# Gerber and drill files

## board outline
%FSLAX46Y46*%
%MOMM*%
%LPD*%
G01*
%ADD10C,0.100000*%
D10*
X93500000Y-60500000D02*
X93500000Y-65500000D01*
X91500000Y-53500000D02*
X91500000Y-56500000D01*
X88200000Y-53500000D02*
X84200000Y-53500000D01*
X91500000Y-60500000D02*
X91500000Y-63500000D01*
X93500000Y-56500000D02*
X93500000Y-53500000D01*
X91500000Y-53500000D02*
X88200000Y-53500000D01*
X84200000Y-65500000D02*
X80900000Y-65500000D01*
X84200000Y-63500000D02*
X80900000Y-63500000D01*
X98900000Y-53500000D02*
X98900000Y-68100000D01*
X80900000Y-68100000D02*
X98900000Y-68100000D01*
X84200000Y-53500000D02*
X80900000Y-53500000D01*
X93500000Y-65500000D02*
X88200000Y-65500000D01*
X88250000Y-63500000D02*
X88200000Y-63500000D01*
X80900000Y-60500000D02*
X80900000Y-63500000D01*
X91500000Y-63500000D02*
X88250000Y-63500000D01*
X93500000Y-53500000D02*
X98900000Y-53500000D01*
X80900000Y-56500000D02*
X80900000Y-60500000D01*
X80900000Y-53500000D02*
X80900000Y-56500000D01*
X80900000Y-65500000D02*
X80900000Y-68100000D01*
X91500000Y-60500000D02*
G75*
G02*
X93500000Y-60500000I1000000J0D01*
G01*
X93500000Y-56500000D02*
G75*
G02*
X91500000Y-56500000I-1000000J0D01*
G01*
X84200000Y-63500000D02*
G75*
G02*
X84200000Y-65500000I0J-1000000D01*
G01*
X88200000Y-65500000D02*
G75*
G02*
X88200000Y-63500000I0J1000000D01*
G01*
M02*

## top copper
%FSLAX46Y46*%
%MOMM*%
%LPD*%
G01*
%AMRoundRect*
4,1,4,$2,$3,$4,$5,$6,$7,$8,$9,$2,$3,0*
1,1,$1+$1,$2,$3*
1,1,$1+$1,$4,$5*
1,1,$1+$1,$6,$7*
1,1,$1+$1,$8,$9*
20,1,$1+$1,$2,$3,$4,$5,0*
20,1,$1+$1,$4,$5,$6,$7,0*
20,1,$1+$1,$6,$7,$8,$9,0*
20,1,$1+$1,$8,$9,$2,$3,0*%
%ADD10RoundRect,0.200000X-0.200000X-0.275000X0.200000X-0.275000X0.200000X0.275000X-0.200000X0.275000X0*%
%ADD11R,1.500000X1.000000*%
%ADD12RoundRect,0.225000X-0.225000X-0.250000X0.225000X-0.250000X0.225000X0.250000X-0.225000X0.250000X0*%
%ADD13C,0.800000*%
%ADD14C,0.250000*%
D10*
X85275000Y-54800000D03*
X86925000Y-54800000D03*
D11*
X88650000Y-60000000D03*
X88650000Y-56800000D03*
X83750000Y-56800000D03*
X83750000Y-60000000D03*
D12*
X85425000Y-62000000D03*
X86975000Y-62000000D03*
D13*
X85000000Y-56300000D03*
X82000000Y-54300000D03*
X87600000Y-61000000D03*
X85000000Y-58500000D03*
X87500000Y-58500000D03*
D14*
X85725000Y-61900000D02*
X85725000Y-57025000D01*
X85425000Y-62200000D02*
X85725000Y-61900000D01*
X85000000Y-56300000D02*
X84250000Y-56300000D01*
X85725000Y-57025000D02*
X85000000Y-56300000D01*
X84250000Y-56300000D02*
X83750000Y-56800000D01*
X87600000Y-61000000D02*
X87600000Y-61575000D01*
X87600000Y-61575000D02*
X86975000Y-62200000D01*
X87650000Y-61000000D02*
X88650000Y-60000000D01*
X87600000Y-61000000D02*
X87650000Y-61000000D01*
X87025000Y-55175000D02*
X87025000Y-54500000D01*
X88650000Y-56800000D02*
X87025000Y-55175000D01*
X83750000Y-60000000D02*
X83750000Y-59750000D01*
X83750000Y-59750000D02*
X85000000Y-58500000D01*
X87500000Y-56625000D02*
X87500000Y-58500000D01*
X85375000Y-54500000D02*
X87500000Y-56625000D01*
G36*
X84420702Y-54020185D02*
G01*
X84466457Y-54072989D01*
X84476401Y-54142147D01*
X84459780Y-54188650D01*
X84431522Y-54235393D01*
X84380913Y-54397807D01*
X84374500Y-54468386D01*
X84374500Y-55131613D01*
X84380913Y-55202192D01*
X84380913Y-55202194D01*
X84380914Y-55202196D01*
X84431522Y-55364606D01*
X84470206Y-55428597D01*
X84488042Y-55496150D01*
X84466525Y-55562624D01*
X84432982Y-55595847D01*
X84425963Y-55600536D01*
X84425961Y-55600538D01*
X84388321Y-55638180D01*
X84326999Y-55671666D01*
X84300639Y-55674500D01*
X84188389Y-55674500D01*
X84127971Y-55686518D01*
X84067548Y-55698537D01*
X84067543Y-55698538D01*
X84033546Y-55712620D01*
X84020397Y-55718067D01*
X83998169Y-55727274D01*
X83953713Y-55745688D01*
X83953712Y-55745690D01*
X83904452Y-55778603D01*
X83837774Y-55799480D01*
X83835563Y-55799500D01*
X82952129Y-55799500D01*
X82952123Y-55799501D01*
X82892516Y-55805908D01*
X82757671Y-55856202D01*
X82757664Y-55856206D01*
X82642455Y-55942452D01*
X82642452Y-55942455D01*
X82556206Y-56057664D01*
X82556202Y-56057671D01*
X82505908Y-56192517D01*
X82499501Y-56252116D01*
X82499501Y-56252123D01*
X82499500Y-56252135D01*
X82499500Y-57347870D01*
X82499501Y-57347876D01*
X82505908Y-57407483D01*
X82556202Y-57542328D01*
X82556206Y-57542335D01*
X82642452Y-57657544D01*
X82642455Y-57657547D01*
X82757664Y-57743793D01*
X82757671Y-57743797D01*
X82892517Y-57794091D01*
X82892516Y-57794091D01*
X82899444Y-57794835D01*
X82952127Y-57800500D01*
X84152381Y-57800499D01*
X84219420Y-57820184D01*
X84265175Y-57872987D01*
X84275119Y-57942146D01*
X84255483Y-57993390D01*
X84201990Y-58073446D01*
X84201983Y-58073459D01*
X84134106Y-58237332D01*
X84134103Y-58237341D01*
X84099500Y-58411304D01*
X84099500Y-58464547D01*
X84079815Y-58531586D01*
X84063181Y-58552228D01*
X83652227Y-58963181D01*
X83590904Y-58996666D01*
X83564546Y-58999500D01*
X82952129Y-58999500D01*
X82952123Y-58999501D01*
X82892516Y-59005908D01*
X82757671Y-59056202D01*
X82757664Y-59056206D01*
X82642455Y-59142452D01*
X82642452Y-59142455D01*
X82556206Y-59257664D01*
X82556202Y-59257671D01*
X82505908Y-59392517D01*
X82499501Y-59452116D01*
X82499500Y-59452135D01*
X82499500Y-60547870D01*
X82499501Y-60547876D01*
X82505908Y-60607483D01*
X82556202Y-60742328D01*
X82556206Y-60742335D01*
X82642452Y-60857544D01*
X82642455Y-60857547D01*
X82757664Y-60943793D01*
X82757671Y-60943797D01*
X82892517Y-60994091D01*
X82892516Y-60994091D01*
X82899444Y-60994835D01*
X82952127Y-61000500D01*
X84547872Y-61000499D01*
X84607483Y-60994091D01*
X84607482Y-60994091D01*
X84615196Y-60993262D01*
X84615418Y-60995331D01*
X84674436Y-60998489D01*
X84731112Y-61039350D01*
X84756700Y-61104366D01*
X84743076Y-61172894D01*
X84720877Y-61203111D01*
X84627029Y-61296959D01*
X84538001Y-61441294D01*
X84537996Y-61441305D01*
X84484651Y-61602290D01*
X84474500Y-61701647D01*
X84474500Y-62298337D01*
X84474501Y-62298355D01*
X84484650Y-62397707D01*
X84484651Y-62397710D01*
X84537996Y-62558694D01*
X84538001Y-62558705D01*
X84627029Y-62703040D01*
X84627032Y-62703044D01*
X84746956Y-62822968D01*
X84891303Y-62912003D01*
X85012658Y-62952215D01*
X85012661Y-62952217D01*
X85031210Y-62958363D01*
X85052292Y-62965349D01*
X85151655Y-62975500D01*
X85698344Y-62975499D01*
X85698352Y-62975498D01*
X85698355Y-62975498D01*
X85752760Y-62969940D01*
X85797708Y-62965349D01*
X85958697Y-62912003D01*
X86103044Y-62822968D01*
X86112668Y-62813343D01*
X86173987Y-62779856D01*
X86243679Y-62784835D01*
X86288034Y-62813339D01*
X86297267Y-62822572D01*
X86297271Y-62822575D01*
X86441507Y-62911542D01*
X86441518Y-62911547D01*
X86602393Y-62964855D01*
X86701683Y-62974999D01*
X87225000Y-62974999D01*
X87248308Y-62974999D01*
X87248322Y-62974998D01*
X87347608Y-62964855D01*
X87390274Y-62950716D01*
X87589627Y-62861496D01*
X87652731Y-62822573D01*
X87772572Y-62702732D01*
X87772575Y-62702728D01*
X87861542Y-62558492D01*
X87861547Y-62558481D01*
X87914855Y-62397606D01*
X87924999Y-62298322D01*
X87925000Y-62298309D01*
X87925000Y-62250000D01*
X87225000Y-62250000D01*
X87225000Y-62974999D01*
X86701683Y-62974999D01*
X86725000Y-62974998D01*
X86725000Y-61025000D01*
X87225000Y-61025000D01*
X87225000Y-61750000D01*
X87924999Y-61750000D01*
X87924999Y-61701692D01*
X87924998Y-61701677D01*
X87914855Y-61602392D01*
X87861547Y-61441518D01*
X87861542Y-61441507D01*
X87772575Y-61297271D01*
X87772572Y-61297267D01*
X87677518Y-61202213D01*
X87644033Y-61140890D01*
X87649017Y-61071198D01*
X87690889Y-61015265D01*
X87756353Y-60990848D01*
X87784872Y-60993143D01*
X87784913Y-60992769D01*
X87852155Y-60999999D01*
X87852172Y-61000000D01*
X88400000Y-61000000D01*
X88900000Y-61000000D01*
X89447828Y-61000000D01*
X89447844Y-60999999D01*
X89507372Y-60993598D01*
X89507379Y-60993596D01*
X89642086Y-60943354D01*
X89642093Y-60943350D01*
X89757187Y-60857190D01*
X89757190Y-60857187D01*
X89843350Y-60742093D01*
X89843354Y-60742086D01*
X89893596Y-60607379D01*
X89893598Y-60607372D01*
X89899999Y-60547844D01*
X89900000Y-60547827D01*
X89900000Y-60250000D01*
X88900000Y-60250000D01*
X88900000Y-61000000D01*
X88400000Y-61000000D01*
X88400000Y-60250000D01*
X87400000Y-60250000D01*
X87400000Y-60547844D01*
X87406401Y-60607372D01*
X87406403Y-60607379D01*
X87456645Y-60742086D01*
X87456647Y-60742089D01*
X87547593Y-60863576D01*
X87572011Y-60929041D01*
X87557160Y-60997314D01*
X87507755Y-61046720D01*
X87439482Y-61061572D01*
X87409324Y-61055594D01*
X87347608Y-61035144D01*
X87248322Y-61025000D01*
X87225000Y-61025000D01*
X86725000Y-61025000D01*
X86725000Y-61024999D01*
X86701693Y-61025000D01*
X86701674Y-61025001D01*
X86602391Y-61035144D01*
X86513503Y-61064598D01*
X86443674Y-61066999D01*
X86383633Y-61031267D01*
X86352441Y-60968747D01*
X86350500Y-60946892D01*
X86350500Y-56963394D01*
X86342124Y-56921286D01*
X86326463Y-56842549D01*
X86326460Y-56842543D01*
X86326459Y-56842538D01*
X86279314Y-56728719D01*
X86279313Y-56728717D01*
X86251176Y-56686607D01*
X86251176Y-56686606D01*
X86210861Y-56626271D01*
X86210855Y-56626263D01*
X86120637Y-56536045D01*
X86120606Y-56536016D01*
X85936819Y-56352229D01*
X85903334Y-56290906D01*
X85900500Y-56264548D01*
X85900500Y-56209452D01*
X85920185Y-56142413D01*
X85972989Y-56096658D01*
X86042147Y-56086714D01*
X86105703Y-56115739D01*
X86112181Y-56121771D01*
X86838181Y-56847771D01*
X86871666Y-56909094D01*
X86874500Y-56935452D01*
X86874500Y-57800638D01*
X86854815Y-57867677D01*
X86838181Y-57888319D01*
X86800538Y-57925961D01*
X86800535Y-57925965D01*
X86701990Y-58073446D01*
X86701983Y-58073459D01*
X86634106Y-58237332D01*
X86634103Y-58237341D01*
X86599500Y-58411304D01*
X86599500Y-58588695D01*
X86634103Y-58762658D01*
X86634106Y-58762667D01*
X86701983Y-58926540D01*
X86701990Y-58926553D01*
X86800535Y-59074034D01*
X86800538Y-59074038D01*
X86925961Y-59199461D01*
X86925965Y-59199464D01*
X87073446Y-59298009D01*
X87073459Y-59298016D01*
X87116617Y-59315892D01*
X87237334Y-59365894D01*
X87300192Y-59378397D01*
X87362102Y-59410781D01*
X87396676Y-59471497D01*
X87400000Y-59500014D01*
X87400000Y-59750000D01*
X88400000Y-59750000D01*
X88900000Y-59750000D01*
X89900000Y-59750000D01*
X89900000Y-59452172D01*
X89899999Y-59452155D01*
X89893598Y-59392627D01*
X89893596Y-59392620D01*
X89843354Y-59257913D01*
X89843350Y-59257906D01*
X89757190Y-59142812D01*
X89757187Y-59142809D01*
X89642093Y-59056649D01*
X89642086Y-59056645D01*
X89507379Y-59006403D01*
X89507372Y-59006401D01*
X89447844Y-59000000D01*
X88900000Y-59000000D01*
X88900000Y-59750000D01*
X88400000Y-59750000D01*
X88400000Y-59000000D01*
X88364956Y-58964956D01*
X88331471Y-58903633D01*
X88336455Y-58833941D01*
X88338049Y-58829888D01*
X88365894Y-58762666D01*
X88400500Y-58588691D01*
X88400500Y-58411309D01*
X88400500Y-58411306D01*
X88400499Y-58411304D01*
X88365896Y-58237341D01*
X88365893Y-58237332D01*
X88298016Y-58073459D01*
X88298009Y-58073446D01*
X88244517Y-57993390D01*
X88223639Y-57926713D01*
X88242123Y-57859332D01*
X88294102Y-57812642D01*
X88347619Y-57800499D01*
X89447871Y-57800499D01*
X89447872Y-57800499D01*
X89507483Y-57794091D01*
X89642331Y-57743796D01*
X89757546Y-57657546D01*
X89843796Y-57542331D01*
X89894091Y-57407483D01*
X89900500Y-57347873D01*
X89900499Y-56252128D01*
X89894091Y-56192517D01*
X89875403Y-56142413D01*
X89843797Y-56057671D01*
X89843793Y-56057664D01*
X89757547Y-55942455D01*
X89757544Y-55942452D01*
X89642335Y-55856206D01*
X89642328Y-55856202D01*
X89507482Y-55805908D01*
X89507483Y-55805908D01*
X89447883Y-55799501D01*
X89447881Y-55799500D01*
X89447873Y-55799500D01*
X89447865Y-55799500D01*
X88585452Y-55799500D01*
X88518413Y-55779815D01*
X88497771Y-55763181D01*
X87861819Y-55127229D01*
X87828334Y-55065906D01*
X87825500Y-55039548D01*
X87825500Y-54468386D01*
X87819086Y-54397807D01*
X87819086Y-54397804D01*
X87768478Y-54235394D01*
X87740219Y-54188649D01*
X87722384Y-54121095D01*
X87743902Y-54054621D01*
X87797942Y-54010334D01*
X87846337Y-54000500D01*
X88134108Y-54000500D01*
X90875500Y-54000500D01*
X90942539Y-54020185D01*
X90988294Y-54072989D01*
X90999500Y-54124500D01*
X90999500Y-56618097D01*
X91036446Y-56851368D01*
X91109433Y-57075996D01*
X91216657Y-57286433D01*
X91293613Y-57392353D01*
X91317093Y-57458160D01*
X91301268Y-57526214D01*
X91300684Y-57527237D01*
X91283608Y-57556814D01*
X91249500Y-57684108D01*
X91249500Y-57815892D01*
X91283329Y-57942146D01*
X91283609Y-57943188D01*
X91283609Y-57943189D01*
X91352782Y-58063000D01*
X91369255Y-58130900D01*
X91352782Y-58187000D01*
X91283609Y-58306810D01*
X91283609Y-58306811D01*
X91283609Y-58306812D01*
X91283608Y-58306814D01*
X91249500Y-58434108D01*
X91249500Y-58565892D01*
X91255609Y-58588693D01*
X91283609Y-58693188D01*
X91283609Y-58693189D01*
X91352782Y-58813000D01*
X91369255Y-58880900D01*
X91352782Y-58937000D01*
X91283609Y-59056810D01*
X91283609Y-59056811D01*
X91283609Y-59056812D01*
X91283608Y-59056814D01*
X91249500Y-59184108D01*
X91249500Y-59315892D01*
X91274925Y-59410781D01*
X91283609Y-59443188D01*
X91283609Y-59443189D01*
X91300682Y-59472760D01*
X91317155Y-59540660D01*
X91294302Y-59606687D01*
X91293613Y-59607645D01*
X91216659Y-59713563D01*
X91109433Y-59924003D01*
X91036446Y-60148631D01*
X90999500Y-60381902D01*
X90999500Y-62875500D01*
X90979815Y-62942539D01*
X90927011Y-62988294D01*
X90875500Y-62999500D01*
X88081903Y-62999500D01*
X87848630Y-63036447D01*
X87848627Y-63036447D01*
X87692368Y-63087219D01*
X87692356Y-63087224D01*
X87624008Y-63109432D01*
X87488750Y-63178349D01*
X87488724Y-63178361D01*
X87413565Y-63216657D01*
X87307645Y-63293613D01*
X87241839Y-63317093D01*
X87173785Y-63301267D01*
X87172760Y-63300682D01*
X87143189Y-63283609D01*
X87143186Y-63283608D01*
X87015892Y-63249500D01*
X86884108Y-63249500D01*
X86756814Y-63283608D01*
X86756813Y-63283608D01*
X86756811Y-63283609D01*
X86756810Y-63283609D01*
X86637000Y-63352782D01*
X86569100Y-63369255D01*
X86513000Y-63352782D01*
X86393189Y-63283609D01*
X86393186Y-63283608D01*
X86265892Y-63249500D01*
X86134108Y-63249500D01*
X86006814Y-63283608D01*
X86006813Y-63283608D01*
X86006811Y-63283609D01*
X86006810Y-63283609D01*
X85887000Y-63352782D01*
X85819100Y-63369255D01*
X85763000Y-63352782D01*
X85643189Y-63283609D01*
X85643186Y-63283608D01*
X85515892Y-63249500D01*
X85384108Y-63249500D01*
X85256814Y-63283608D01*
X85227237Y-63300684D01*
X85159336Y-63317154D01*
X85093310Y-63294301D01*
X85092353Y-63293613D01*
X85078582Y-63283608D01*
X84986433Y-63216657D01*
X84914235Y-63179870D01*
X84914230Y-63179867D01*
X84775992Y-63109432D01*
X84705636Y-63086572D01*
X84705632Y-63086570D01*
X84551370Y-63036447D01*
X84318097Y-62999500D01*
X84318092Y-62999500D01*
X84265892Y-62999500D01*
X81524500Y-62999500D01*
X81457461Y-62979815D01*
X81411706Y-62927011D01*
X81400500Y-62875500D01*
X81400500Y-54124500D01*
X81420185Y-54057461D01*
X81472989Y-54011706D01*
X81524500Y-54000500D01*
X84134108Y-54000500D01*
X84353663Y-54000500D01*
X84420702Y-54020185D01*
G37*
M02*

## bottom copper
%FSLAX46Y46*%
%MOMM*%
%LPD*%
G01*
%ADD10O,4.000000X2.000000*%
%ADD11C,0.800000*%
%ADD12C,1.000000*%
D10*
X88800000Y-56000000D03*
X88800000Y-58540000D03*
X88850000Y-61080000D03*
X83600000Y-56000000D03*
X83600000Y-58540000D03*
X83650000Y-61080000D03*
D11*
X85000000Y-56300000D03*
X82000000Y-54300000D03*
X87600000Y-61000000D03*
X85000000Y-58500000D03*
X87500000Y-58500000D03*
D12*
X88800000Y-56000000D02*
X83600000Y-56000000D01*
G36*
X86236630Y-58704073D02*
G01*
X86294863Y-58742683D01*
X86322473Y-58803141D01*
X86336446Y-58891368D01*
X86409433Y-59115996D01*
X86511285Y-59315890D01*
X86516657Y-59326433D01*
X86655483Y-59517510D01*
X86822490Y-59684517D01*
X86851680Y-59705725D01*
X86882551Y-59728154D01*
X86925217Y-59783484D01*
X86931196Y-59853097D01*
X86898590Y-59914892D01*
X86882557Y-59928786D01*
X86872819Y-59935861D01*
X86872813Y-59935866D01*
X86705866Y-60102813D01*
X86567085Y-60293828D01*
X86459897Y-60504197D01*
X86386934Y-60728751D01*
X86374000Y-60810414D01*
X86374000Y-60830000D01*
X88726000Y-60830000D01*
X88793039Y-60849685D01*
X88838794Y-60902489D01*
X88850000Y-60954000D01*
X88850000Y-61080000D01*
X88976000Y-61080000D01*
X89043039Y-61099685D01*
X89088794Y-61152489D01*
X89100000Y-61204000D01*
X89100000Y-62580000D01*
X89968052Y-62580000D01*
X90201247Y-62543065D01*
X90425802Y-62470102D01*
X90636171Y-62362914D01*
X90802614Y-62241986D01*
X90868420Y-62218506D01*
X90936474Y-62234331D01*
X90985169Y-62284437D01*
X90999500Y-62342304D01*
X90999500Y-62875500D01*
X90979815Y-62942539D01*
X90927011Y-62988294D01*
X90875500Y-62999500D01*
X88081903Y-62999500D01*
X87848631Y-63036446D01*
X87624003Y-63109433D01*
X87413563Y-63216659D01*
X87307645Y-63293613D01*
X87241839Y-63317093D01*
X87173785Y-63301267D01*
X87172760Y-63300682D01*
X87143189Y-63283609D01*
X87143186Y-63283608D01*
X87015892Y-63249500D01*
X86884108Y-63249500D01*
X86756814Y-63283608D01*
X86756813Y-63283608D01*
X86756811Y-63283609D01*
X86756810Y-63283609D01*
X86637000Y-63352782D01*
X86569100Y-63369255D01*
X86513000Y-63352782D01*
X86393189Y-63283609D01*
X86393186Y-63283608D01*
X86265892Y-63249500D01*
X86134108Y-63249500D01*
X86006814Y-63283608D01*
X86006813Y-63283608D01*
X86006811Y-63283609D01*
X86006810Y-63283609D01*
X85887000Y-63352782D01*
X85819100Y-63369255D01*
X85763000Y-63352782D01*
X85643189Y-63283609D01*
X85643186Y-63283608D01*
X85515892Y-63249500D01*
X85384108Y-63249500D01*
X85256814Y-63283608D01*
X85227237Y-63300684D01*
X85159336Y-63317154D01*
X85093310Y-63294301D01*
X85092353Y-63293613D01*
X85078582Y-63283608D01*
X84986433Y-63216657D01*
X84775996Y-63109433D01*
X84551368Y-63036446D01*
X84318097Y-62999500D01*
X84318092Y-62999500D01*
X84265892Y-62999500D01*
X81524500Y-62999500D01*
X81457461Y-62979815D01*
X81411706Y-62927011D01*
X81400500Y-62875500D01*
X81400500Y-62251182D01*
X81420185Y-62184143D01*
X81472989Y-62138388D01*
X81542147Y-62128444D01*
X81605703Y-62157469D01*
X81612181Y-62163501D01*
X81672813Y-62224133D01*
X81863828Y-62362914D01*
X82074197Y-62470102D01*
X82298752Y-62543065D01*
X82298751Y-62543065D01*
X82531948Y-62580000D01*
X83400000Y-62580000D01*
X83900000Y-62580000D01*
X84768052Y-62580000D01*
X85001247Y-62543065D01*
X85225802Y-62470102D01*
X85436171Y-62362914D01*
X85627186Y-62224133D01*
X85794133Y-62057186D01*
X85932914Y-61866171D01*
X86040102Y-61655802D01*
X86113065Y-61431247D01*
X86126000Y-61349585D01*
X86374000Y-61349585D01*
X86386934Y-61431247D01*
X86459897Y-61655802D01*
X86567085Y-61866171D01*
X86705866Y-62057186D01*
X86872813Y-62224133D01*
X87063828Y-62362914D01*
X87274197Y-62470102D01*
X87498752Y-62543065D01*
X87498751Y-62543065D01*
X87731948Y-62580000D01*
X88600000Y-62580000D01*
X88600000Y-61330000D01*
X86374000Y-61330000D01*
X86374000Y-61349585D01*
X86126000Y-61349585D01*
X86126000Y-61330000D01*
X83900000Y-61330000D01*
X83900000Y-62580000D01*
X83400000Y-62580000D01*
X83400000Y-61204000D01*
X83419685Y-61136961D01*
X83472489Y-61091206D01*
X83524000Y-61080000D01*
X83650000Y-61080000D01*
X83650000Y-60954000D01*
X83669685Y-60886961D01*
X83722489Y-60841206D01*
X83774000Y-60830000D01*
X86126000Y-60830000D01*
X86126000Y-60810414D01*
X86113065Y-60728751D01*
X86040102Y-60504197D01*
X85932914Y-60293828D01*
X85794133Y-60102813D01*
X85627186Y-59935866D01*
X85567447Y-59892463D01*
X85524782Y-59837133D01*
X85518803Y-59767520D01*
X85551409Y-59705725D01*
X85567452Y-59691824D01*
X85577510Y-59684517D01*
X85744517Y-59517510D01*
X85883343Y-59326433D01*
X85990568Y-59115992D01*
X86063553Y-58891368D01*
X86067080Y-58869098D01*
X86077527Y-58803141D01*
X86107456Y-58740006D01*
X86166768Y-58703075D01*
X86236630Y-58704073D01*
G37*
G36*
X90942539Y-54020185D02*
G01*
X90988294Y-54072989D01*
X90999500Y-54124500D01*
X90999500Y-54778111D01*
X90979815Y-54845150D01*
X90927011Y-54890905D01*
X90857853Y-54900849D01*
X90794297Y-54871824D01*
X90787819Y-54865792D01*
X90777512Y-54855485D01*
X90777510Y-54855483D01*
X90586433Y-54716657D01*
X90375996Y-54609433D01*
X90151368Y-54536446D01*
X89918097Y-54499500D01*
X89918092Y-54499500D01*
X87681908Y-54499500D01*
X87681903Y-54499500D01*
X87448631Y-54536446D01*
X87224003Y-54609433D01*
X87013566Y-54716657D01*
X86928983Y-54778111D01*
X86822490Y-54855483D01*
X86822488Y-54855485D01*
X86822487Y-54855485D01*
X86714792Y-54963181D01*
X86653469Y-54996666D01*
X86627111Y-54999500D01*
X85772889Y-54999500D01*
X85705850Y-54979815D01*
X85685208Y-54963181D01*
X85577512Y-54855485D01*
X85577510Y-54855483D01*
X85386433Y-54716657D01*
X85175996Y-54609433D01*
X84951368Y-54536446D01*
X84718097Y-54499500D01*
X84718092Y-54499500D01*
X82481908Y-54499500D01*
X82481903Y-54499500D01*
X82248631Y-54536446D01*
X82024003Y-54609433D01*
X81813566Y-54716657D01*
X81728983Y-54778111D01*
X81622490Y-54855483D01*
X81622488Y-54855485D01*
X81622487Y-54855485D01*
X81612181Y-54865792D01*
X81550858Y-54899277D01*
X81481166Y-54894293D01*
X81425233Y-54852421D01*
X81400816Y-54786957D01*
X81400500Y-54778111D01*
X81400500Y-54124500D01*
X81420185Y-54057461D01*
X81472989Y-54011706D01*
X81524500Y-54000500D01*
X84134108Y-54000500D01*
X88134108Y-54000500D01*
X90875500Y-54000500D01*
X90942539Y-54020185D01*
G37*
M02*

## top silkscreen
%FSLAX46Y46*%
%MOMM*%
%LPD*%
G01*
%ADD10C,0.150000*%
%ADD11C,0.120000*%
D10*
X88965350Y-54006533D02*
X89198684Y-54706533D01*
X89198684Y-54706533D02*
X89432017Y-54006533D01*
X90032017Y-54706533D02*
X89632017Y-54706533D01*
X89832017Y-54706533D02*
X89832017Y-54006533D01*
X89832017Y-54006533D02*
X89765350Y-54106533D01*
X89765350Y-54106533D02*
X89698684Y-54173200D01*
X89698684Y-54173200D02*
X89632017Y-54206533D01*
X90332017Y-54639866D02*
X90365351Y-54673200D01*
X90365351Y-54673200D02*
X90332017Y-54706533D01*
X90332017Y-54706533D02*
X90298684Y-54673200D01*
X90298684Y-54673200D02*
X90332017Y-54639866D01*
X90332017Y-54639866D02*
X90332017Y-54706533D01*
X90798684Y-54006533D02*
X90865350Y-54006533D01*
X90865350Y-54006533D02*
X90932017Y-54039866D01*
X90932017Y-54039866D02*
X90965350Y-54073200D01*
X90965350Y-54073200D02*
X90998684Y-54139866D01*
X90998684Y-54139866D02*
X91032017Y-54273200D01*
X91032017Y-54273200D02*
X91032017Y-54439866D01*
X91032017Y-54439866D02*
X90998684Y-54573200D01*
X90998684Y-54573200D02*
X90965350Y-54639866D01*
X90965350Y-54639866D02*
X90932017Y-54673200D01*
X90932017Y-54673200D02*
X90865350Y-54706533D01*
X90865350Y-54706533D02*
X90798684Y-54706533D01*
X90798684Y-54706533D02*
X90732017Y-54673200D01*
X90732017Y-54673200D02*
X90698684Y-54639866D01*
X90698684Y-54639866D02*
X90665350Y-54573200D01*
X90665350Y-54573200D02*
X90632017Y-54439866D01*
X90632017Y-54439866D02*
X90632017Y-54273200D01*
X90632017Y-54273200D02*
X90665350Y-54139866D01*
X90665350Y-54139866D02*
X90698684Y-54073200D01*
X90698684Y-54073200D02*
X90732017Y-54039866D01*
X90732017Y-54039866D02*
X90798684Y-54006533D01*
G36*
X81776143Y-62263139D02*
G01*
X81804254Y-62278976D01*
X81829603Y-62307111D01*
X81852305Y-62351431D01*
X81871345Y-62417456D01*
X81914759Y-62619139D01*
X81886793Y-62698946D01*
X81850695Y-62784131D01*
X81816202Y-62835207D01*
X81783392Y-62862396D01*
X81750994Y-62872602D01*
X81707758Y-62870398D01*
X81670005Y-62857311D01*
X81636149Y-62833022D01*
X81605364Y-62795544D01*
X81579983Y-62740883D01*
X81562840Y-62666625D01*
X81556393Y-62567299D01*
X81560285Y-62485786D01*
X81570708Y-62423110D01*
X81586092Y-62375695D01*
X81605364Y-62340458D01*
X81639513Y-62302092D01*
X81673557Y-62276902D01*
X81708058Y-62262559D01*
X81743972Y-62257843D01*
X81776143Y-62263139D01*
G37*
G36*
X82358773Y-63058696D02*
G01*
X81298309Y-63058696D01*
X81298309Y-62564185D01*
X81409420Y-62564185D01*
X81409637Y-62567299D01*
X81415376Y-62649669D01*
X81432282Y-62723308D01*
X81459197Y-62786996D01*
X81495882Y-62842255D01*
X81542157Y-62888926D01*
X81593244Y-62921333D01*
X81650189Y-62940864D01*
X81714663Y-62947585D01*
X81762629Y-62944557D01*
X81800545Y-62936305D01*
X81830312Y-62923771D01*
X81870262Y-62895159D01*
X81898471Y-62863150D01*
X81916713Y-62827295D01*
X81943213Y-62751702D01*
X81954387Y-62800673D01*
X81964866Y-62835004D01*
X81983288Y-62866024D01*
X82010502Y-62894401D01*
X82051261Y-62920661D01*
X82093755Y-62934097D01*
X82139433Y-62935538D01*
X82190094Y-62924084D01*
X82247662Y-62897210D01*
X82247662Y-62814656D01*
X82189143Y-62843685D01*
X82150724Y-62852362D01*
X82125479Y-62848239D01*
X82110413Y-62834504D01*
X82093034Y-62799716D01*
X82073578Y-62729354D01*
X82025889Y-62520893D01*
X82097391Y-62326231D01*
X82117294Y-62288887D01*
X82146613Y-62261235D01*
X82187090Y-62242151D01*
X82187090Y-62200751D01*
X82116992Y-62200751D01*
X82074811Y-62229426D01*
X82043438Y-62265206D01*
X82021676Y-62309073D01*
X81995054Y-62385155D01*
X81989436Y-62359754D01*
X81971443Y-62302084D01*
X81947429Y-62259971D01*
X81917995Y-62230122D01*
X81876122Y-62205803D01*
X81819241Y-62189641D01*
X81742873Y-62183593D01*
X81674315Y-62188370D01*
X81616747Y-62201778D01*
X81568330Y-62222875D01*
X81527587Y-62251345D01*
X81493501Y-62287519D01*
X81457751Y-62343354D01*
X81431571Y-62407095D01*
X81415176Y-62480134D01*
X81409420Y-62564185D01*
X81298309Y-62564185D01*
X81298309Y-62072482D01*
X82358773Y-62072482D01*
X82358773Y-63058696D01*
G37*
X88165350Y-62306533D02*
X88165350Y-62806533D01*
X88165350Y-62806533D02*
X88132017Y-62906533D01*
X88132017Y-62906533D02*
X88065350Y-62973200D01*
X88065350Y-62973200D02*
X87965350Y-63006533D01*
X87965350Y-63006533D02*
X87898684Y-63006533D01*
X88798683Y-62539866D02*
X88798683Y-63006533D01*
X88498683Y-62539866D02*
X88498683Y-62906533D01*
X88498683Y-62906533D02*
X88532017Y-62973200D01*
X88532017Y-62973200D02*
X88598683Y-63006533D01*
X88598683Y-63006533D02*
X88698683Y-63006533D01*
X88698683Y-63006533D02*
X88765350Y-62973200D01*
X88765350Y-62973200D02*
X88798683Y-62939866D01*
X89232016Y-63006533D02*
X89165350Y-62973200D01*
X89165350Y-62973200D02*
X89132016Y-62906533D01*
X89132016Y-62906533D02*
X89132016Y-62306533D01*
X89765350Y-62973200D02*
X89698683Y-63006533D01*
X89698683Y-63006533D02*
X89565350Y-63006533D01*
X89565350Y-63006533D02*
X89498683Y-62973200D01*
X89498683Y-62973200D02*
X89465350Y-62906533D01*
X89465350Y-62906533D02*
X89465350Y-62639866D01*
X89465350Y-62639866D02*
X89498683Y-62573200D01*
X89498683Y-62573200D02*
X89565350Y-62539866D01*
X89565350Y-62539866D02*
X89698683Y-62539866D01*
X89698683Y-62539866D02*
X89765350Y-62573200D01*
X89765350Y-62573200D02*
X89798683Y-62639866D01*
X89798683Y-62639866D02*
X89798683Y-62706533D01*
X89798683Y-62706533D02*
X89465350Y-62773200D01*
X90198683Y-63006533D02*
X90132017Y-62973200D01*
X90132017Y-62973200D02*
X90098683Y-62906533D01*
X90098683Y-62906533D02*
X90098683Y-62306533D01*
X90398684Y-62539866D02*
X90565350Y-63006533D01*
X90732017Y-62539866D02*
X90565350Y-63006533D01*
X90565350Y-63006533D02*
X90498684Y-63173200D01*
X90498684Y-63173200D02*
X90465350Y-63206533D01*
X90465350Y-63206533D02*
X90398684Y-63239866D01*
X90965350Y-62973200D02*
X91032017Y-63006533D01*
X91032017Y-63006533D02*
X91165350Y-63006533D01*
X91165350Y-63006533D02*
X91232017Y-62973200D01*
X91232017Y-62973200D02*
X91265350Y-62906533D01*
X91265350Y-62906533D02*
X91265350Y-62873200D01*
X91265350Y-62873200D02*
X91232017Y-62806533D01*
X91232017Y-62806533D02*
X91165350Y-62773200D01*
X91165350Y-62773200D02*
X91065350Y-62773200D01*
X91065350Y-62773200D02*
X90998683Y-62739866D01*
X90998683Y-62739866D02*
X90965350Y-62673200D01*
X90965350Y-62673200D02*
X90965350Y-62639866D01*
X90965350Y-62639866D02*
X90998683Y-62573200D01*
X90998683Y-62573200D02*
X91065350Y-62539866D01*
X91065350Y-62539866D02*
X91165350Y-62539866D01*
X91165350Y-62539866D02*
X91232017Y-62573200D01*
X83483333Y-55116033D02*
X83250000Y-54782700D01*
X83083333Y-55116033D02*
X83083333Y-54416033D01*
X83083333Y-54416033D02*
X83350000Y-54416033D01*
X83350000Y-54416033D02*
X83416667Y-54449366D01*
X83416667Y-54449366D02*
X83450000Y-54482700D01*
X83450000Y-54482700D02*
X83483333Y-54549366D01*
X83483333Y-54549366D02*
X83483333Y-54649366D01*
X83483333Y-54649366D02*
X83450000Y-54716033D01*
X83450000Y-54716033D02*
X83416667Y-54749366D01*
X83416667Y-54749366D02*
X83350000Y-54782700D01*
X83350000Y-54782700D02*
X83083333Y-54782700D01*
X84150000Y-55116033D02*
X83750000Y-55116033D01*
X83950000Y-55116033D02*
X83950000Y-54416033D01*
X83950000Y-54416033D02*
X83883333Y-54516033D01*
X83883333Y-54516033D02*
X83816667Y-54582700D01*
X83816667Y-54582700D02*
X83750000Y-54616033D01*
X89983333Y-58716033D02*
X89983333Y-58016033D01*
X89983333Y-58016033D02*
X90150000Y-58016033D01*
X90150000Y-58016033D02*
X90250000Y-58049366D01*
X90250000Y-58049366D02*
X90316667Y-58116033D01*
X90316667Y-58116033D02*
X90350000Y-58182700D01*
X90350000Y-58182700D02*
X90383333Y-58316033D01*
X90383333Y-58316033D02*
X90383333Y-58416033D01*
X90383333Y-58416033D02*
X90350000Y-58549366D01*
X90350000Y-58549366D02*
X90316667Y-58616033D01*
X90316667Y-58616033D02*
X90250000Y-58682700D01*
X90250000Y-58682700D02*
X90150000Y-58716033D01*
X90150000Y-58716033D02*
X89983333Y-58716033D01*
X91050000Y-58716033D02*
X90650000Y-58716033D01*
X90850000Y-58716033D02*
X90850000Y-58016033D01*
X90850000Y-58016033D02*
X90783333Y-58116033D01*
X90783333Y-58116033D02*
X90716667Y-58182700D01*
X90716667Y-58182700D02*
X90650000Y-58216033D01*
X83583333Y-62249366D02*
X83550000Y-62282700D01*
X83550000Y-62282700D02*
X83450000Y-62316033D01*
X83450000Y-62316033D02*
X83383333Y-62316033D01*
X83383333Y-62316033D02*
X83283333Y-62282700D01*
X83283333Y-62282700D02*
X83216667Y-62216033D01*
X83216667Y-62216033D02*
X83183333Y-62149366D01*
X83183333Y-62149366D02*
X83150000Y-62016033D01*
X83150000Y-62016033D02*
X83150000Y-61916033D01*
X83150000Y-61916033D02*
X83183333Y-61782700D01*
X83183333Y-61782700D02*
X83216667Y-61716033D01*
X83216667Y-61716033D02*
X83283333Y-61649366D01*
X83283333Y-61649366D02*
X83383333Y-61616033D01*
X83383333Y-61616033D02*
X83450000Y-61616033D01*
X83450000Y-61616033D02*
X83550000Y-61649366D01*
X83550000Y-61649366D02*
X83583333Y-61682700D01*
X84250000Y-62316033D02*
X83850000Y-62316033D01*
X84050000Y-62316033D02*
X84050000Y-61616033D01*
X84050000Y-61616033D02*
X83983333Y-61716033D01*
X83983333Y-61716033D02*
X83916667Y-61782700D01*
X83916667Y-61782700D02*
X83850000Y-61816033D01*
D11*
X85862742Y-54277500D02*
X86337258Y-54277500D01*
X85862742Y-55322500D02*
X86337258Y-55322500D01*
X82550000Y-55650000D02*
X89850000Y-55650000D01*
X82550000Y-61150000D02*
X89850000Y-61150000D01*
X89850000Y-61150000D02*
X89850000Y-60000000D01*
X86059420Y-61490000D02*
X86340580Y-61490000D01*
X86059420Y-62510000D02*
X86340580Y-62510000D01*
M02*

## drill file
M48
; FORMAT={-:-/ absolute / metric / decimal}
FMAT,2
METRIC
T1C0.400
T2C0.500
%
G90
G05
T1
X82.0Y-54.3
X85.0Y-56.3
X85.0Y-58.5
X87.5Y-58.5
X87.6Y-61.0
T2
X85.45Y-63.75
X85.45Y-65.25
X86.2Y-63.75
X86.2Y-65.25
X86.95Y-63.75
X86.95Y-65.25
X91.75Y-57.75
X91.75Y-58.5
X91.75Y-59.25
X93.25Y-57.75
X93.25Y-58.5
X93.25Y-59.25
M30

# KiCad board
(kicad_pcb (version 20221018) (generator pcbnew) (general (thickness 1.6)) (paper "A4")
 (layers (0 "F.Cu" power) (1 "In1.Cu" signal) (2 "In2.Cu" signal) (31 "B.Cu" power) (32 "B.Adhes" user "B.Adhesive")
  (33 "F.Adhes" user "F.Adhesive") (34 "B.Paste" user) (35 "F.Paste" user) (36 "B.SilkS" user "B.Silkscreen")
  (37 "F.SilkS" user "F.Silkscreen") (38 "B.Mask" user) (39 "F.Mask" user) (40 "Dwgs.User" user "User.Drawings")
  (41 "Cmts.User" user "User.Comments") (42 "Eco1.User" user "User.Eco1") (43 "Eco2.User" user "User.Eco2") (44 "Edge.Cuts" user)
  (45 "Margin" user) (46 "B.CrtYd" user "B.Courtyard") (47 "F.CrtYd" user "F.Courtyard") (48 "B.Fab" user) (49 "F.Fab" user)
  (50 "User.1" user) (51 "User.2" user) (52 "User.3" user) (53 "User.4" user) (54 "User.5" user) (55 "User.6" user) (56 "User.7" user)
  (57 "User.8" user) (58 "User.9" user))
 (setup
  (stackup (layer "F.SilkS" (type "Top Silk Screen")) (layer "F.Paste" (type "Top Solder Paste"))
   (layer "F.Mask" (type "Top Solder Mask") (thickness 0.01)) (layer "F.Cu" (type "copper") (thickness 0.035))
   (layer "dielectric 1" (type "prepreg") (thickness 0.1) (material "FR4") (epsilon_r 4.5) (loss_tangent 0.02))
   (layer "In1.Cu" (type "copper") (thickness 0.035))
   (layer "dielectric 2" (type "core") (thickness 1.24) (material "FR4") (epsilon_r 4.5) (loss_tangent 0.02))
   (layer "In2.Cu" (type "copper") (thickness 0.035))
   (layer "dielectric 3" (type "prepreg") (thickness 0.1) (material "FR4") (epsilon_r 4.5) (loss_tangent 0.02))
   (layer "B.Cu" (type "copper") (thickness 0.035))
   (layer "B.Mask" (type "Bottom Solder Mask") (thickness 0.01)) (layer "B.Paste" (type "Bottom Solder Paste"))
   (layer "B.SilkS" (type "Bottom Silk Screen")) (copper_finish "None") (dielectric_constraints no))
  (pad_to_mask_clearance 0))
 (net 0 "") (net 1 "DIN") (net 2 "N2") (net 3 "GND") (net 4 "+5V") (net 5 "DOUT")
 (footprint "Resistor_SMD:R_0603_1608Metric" (layer "F.Cu") (at 86.1 54.8)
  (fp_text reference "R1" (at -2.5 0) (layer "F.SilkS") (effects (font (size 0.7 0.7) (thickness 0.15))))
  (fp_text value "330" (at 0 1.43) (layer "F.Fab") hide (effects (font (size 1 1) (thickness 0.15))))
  (fp_line (start -0.237258 -0.5225) (end 0.237258 -0.5225) (stroke (width 0.12) (type solid)) (layer "F.SilkS"))
  (fp_line (start -0.237258 0.5225) (end 0.237258 0.5225) (stroke (width 0.12) (type solid)) (layer "F.SilkS"))
  (pad "1" smd roundrect (at -0.825 0) (size 0.8 0.95) (layers "F.Cu" "F.Paste" "F.Mask") (roundrect_rratio 0.25) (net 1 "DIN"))
  (pad "2" smd roundrect (at 0.825 0) (size 0.8 0.95) (layers "F.Cu" "F.Paste" "F.Mask") (roundrect_rratio 0.25) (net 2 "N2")))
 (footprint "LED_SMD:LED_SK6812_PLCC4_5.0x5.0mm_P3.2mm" (layer "F.Cu") (at 86.2 58.4)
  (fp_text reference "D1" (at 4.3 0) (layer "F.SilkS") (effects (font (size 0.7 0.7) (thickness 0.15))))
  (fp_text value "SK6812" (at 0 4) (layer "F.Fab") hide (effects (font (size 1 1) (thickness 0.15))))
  (fp_line (start -3.65 -2.75) (end 3.65 -2.75) (stroke (width 0.12) (type solid)) (layer "F.SilkS"))
  (fp_line (start -3.65 2.75) (end 3.65 2.75) (stroke (width 0.12) (type solid)) (layer "F.SilkS"))
  (fp_line (start 3.65 2.75) (end 3.65 1.6) (stroke (width 0.12) (type solid)) (layer "F.SilkS"))
  (pad "1" smd rect (at 2.45 1.6) (size 1.5 1) (layers "F.Cu" "F.Paste" "F.Mask") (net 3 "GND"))
  (pad "2" smd rect (at 2.45 -1.6) (size 1.5 1) (layers "F.Cu" "F.Paste" "F.Mask") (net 2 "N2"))
  (pad "3" smd rect (at -2.45 -1.6) (size 1.5 1) (layers "F.Cu" "F.Paste" "F.Mask") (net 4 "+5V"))
  (pad "4" smd rect (at -2.45 1.6) (size 1.5 1) (layers "F.Cu" "F.Paste" "F.Mask") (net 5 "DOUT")))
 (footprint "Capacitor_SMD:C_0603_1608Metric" (layer "F.Cu") (at 86.2 62)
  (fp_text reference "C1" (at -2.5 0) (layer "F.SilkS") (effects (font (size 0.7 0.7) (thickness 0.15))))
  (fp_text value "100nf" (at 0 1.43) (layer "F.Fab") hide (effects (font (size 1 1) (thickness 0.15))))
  (fp_line (start -0.14058 -0.51) (end 0.14058 -0.51) (stroke (width 0.12) (type solid)) (layer "F.SilkS"))
  (fp_line (start -0.14058 0.51) (end 0.14058 0.51) (stroke (width 0.12) (type solid)) (layer "F.SilkS"))
  (pad "1" smd roundrect (at -0.775 0) (size 0.9 0.95) (layers "F.Cu" "F.Paste" "F.Mask") (roundrect_rratio 0.25) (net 4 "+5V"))
  (pad "2" smd roundrect (at 0.775 0) (size 0.9 0.95) (layers "F.Cu" "F.Paste" "F.Mask") (roundrect_rratio 0.25) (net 3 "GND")))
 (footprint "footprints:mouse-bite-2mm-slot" (layer "F.Cu") (at 92.5 58.5 90)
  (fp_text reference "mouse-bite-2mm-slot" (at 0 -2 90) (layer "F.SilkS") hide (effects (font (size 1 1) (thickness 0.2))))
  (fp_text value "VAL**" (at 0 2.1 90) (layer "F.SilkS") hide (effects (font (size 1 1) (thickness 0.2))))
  (fp_arc (start -2 -1) (mid -1 0) (end -2 1) (stroke (width 0.1) (type solid)) (layer "Edge.Cuts"))
  (fp_arc (start 2 1) (mid 1 0) (end 2 -1) (stroke (width 0.1) (type solid)) (layer "Edge.Cuts"))
  (pad "" np_thru_hole circle (at -0.75 -0.75 90) (size 0.5 0.5) (drill 0.5) (layers "*.Cu" "*.Mask"))
  (pad "" np_thru_hole circle (at -0.75 0.75 90) (size 0.5 0.5) (drill 0.5) (layers "*.Cu" "*.Mask"))
  (pad "" np_thru_hole circle (at 0 -0.75 90) (size 0.5 0.5) (drill 0.5) (layers "*.Cu" "*.Mask"))
  (pad "" np_thru_hole circle (at 0 0.75 90) (size 0.5 0.5) (drill 0.5) (layers "*.Cu" "*.Mask"))
  (pad "" np_thru_hole circle (at 0.75 -0.75 90) (size 0.5 0.5) (drill 0.5) (layers "*.Cu" "*.Mask"))
  (pad "" np_thru_hole circle (at 0.75 0.75 90) (size 0.5 0.5) (drill 0.5) (layers "*.Cu" "*.Mask")))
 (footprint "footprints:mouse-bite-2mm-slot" (layer "F.Cu") (at 86.2 64.5)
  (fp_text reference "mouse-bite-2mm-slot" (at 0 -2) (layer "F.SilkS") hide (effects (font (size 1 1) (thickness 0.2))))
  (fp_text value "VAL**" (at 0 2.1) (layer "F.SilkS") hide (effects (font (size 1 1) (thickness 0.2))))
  (fp_arc (start -2 -1) (mid -1 0) (end -2 1) (stroke (width 0.1) (type solid)) (layer "Edge.Cuts"))
  (fp_arc (start 2 1) (mid 1 0) (end 2 -1) (stroke (width 0.1) (type solid)) (layer "Edge.Cuts"))
  (pad "" np_thru_hole circle (at -0.75 -0.75) (size 0.5 0.5) (drill 0.5) (layers "*.Cu" "*.Mask"))
  (pad "" np_thru_hole circle (at -0.75 0.75) (size 0.5 0.5) (drill 0.5) (layers "*.Cu" "*.Mask"))
  (pad "" np_thru_hole circle (at 0 -0.75) (size 0.5 0.5) (drill 0.5) (layers "*.Cu" "*.Mask"))
  (pad "" np_thru_hole circle (at 0 0.75) (size 0.5 0.5) (drill 0.5) (layers "*.Cu" "*.Mask"))
  (pad "" np_thru_hole circle (at 0.75 -0.75) (size 0.5 0.5) (drill 0.5) (layers "*.Cu" "*.Mask"))
  (pad "" np_thru_hole circle (at 0.75 0.75) (size 0.5 0.5) (drill 0.5) (layers "*.Cu" "*.Mask")))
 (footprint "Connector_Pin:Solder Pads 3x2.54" (layer "B.Cu") (at 88.8 59.6 180)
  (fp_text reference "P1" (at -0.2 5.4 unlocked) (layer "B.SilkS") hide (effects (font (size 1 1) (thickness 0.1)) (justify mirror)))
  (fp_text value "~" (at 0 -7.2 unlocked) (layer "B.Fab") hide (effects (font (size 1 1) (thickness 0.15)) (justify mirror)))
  (pad "1" connect oval (at 0 3.6 180) (size 4 2) (layers "B.Cu" "B.Mask") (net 4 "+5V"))
  (pad "2" connect oval (at 0 1.06 180) (size 4 2) (layers "B.Cu" "B.Mask") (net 1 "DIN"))
  (pad "3" connect oval (at -0.05 -1.48 180) (size 4 2) (layers "B.Cu" "B.Mask") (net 3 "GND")))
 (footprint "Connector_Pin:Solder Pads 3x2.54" (layer "B.Cu") (at 83.6 59.6 180)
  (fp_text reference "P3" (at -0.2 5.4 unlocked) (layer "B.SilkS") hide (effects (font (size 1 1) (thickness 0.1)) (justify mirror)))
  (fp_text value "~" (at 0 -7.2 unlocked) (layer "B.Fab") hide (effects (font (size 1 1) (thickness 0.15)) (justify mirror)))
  (pad "1" connect oval (at 0 3.6 180) (size 4 2) (layers "B.Cu" "B.Mask") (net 4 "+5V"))
  (pad "2" connect oval (at 0 1.06 180) (size 4 2) (layers "B.Cu" "B.Mask") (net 5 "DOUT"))
  (pad "3" connect oval (at -0.05 -1.48 180) (size 4 2) (layers "B.Cu" "B.Mask") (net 3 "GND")))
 (gr_line (start 93.5 60.5) (end 93.5 65.5) (stroke (width 0.1) (type default)) (layer "Edge.Cuts"))
 (gr_line (start 91.5 53.5) (end 91.5 56.5) (stroke (width 0.1) (type default)) (layer "Edge.Cuts"))
 (gr_line (start 88.2 53.5) (end 84.2 53.5) (stroke (width 0.1) (type default)) (layer "Edge.Cuts"))
 (gr_line (start 91.5 60.5) (end 91.5 63.5) (stroke (width 0.1) (type default)) (layer "Edge.Cuts"))
 (gr_line (start 93.5 56.5) (end 93.5 53.5) (stroke (width 0.1) (type default)) (layer "Edge.Cuts"))
 (gr_line (start 91.5 53.5) (end 88.2 53.5) (stroke (width 0.1) (type default)) (layer "Edge.Cuts"))
 (gr_line (start 84.2 65.5) (end 80.9 65.5) (stroke (width 0.1) (type default)) (layer "Edge.Cuts"))
 (gr_line (start 84.2 63.5) (end 80.9 63.5) (stroke (width 0.1) (type default)) (layer "Edge.Cuts"))
 (gr_line (start 98.9 53.5) (end 98.9 68.1) (stroke (width 0.1) (type default)) (layer "Edge.Cuts"))
 (gr_line (start 80.9 68.1) (end 98.9 68.1) (stroke (width 0.1) (type default)) (layer "Edge.Cuts"))
 (gr_line (start 84.2 53.5) (end 80.9 53.5) (stroke (width 0.1) (type default)) (layer "Edge.Cuts"))
 (gr_line (start 93.5 65.5) (end 88.2 65.5) (stroke (width 0.1) (type default)) (layer "Edge.Cuts"))
 (gr_line (start 88.25 63.5) (end 88.2 63.5) (stroke (width 0.1) (type default)) (layer "Edge.Cuts"))
 (gr_line (start 80.9 60.5) (end 80.9 63.5) (stroke (width 0.1) (type default)) (layer "Edge.Cuts"))
 (gr_line (start 91.5 63.5) (end 88.25 63.5) (stroke (width 0.1) (type default)) (layer "Edge.Cuts"))
 (gr_line (start 93.5 53.5) (end 98.9 53.5) (stroke (width 0.1) (type default)) (layer "Edge.Cuts"))
 (gr_line (start 80.9 56.5) (end 80.9 60.5) (stroke (width 0.1) (type default)) (layer "Edge.Cuts"))
 (gr_line (start 80.9 53.5) (end 80.9 56.5) (stroke (width 0.1) (type default)) (layer "Edge.Cuts"))
 (gr_line (start 80.9 65.5) (end 80.9 68.1) (stroke (width 0.1) (type default)) (layer "Edge.Cuts"))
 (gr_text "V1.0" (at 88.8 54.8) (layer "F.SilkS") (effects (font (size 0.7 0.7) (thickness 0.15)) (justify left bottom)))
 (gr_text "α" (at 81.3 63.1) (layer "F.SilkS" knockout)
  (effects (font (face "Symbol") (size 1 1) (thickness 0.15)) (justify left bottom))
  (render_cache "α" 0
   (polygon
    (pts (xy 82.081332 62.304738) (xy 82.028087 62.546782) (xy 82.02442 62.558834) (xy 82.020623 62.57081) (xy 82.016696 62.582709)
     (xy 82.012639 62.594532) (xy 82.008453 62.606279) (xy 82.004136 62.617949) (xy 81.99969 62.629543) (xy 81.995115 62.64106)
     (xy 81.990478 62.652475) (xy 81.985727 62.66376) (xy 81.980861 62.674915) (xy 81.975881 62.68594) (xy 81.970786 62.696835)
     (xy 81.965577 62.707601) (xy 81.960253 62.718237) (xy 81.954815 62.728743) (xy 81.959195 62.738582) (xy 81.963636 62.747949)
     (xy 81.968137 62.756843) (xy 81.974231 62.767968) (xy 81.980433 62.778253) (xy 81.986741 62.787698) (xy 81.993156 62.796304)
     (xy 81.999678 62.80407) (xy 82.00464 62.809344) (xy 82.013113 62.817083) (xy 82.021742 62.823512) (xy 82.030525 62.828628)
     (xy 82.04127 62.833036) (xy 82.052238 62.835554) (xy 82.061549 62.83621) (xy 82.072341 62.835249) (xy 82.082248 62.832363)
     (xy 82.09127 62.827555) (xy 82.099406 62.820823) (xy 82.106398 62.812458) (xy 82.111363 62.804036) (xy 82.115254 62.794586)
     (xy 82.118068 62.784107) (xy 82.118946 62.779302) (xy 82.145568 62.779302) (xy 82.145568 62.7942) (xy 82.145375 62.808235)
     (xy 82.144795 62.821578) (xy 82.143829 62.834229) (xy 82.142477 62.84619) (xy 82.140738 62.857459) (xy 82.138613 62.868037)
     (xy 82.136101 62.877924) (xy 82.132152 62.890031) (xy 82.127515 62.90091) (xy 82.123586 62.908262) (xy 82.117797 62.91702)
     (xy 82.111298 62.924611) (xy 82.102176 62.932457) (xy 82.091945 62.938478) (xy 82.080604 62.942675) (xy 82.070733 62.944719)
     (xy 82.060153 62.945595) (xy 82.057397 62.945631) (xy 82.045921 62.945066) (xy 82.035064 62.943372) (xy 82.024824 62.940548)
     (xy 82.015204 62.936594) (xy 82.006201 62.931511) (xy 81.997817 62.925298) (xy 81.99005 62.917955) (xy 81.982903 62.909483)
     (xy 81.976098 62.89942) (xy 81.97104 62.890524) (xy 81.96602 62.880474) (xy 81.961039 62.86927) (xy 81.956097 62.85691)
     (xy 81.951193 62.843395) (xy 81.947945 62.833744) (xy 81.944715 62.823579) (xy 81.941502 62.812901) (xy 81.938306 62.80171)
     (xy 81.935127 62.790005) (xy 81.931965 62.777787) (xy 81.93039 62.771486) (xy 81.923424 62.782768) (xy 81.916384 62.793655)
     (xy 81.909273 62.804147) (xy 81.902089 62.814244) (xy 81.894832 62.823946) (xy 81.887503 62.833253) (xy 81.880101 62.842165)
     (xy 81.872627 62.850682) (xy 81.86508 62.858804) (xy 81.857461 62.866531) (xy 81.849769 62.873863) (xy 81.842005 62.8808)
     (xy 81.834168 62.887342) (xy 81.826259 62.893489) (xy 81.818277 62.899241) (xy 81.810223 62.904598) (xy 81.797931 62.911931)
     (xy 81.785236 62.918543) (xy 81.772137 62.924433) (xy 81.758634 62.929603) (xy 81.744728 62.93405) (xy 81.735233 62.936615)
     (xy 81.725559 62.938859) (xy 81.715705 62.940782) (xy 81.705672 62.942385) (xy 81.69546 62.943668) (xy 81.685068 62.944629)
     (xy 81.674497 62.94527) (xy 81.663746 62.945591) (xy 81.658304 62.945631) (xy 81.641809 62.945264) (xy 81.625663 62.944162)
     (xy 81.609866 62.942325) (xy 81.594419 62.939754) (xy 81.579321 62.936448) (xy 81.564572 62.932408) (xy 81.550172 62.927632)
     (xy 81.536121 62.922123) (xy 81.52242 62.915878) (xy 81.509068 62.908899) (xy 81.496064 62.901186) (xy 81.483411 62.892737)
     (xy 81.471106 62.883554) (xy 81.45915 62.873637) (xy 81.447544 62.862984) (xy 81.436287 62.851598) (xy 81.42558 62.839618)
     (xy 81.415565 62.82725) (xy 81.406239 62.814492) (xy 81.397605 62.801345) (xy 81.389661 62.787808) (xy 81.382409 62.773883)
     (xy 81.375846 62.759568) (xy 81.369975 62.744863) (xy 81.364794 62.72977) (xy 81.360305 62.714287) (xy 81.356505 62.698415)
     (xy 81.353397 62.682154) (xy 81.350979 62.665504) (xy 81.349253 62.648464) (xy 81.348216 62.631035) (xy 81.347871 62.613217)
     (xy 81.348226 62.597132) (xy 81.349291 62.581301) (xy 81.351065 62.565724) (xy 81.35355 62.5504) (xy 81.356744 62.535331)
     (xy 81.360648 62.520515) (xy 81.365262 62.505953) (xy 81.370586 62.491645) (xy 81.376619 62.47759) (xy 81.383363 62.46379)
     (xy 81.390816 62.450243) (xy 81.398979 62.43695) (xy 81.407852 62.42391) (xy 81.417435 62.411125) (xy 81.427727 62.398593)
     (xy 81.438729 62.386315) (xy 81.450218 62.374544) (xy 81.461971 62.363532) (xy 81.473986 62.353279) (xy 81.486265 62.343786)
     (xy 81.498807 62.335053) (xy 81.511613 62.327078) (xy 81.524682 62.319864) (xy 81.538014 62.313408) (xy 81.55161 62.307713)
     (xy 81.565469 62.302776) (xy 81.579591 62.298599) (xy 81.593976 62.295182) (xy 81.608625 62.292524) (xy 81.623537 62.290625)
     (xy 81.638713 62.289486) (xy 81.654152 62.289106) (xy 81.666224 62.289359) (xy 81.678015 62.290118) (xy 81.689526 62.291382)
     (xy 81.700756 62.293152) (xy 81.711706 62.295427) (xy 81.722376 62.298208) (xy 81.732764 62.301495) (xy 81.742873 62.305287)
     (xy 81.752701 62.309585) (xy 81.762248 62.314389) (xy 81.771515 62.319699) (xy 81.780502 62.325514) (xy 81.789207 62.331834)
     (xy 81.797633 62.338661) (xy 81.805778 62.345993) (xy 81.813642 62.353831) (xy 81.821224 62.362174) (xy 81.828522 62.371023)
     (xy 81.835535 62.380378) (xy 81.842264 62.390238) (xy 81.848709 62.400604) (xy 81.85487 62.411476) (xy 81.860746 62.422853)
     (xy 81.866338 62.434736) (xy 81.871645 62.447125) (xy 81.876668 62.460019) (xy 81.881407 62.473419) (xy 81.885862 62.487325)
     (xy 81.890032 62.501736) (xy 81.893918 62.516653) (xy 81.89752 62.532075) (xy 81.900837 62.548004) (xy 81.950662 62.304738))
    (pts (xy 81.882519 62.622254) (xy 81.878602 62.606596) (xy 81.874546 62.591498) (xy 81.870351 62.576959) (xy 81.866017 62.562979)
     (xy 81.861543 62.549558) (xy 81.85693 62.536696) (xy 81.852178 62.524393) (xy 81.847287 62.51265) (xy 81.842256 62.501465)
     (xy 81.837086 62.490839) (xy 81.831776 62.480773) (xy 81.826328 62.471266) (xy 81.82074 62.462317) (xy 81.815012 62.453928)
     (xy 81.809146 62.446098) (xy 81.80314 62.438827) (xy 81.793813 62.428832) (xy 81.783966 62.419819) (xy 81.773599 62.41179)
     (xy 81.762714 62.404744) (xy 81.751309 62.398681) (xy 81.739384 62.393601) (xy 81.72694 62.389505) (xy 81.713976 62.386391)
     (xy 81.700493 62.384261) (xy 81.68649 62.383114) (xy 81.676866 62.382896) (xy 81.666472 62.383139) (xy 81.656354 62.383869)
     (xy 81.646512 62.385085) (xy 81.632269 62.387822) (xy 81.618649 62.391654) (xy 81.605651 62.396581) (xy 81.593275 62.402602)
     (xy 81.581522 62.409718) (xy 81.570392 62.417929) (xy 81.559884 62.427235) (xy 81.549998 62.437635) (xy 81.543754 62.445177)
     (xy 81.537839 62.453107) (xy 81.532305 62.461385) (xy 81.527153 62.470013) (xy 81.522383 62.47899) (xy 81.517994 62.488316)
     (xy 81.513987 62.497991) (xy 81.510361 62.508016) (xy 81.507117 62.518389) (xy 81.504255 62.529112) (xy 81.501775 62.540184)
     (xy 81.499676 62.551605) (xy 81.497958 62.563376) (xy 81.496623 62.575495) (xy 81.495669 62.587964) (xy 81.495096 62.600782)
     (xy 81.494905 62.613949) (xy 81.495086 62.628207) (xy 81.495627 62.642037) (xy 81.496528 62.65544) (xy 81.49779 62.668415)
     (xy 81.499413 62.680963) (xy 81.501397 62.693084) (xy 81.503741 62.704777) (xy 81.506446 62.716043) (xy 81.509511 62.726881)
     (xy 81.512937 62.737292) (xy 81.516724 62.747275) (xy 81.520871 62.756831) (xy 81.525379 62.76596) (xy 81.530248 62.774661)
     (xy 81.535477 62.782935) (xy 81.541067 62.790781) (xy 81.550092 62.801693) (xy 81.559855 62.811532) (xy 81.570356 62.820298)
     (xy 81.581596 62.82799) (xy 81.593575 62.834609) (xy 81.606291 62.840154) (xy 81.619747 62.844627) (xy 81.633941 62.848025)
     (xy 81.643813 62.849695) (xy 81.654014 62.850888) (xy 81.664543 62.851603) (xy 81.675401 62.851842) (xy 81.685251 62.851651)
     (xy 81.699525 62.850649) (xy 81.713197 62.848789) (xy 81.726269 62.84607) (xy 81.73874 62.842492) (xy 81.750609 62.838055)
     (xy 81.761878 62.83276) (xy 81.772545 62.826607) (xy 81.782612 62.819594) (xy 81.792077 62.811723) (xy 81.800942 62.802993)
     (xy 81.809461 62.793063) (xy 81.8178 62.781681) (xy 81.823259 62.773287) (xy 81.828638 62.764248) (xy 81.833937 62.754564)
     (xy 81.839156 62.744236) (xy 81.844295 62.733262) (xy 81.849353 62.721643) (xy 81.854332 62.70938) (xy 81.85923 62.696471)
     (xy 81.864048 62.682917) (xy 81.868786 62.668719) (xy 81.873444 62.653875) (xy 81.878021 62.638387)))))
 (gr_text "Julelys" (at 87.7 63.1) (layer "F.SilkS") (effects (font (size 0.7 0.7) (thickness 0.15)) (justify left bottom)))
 (segment (start 85.725 61.9) (end 85.725 57.025) (width 0.25) (layer "F.Cu") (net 4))
 (segment (start 85.425 62.2) (end 85.725 61.9) (width 0.25) (layer "F.Cu") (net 4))
 (segment (start 85 56.3) (end 84.25 56.3) (width 0.25) (layer "F.Cu") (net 4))
 (segment (start 85.725 57.025) (end 85 56.3) (width 0.25) (layer "F.Cu") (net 4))
 (segment (start 84.25 56.3) (end 83.75 56.8) (width 0.25) (layer "F.Cu") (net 4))
 (via (at 85 56.3) (size 0.8) (drill 0.4) (layers "F.Cu" "B.Cu") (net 4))
 (segment (start 88.8 56) (end 83.6 56) (width 1) (layer "B.Cu") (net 4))
 (segment (start 87.6 61) (end 87.6 61.575) (width 0.25) (layer "F.Cu") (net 3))
 (segment (start 87.6 61.575) (end 86.975 62.2) (width 0.25) (layer "F.Cu") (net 3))
 (segment (start 87.65 61) (end 88.65 60) (width 0.25) (layer "F.Cu") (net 3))
 (segment (start 87.6 61) (end 87.65 61) (width 0.25) (layer "F.Cu") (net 3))
 (via (at 82 54.3) (size 0.8) (drill 0.4) (layers "F.Cu" "B.Cu") (free) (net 3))
 (via (at 87.6 61) (size 0.8) (drill 0.4) (layers "F.Cu" "B.Cu") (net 3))
 (segment (start 87.025 55.175) (end 87.025 54.5) (width 0.25) (layer "F.Cu") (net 2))
 (segment (start 88.65 56.8) (end 87.025 55.175) (width 0.25) (layer "F.Cu") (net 2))
 (segment (start 83.75 60) (end 83.75 59.75) (width 0.25) (layer "F.Cu") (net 5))
 (segment (start 83.75 59.75) (end 85 58.5) (width 0.25) (layer "F.Cu") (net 5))
 (via (at 85 58.5) (size 0.8) (drill 0.4) (layers "F.Cu" "B.Cu") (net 5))
 (segment (start 87.5 56.625) (end 87.5 58.5) (width 0.25) (layer "F.Cu") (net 1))
 (segment (start 85.375 54.5) (end 87.5 56.625) (width 0.25) (layer "F.Cu") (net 1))
 (via (at 87.5 58.5) (size 0.8) (drill 0.4) (layers "F.Cu" "B.Cu") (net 1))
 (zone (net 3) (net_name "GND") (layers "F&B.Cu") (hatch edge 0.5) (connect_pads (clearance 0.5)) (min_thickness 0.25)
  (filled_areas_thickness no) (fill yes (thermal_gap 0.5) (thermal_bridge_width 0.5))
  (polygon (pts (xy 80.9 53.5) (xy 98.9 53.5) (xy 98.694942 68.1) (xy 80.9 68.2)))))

